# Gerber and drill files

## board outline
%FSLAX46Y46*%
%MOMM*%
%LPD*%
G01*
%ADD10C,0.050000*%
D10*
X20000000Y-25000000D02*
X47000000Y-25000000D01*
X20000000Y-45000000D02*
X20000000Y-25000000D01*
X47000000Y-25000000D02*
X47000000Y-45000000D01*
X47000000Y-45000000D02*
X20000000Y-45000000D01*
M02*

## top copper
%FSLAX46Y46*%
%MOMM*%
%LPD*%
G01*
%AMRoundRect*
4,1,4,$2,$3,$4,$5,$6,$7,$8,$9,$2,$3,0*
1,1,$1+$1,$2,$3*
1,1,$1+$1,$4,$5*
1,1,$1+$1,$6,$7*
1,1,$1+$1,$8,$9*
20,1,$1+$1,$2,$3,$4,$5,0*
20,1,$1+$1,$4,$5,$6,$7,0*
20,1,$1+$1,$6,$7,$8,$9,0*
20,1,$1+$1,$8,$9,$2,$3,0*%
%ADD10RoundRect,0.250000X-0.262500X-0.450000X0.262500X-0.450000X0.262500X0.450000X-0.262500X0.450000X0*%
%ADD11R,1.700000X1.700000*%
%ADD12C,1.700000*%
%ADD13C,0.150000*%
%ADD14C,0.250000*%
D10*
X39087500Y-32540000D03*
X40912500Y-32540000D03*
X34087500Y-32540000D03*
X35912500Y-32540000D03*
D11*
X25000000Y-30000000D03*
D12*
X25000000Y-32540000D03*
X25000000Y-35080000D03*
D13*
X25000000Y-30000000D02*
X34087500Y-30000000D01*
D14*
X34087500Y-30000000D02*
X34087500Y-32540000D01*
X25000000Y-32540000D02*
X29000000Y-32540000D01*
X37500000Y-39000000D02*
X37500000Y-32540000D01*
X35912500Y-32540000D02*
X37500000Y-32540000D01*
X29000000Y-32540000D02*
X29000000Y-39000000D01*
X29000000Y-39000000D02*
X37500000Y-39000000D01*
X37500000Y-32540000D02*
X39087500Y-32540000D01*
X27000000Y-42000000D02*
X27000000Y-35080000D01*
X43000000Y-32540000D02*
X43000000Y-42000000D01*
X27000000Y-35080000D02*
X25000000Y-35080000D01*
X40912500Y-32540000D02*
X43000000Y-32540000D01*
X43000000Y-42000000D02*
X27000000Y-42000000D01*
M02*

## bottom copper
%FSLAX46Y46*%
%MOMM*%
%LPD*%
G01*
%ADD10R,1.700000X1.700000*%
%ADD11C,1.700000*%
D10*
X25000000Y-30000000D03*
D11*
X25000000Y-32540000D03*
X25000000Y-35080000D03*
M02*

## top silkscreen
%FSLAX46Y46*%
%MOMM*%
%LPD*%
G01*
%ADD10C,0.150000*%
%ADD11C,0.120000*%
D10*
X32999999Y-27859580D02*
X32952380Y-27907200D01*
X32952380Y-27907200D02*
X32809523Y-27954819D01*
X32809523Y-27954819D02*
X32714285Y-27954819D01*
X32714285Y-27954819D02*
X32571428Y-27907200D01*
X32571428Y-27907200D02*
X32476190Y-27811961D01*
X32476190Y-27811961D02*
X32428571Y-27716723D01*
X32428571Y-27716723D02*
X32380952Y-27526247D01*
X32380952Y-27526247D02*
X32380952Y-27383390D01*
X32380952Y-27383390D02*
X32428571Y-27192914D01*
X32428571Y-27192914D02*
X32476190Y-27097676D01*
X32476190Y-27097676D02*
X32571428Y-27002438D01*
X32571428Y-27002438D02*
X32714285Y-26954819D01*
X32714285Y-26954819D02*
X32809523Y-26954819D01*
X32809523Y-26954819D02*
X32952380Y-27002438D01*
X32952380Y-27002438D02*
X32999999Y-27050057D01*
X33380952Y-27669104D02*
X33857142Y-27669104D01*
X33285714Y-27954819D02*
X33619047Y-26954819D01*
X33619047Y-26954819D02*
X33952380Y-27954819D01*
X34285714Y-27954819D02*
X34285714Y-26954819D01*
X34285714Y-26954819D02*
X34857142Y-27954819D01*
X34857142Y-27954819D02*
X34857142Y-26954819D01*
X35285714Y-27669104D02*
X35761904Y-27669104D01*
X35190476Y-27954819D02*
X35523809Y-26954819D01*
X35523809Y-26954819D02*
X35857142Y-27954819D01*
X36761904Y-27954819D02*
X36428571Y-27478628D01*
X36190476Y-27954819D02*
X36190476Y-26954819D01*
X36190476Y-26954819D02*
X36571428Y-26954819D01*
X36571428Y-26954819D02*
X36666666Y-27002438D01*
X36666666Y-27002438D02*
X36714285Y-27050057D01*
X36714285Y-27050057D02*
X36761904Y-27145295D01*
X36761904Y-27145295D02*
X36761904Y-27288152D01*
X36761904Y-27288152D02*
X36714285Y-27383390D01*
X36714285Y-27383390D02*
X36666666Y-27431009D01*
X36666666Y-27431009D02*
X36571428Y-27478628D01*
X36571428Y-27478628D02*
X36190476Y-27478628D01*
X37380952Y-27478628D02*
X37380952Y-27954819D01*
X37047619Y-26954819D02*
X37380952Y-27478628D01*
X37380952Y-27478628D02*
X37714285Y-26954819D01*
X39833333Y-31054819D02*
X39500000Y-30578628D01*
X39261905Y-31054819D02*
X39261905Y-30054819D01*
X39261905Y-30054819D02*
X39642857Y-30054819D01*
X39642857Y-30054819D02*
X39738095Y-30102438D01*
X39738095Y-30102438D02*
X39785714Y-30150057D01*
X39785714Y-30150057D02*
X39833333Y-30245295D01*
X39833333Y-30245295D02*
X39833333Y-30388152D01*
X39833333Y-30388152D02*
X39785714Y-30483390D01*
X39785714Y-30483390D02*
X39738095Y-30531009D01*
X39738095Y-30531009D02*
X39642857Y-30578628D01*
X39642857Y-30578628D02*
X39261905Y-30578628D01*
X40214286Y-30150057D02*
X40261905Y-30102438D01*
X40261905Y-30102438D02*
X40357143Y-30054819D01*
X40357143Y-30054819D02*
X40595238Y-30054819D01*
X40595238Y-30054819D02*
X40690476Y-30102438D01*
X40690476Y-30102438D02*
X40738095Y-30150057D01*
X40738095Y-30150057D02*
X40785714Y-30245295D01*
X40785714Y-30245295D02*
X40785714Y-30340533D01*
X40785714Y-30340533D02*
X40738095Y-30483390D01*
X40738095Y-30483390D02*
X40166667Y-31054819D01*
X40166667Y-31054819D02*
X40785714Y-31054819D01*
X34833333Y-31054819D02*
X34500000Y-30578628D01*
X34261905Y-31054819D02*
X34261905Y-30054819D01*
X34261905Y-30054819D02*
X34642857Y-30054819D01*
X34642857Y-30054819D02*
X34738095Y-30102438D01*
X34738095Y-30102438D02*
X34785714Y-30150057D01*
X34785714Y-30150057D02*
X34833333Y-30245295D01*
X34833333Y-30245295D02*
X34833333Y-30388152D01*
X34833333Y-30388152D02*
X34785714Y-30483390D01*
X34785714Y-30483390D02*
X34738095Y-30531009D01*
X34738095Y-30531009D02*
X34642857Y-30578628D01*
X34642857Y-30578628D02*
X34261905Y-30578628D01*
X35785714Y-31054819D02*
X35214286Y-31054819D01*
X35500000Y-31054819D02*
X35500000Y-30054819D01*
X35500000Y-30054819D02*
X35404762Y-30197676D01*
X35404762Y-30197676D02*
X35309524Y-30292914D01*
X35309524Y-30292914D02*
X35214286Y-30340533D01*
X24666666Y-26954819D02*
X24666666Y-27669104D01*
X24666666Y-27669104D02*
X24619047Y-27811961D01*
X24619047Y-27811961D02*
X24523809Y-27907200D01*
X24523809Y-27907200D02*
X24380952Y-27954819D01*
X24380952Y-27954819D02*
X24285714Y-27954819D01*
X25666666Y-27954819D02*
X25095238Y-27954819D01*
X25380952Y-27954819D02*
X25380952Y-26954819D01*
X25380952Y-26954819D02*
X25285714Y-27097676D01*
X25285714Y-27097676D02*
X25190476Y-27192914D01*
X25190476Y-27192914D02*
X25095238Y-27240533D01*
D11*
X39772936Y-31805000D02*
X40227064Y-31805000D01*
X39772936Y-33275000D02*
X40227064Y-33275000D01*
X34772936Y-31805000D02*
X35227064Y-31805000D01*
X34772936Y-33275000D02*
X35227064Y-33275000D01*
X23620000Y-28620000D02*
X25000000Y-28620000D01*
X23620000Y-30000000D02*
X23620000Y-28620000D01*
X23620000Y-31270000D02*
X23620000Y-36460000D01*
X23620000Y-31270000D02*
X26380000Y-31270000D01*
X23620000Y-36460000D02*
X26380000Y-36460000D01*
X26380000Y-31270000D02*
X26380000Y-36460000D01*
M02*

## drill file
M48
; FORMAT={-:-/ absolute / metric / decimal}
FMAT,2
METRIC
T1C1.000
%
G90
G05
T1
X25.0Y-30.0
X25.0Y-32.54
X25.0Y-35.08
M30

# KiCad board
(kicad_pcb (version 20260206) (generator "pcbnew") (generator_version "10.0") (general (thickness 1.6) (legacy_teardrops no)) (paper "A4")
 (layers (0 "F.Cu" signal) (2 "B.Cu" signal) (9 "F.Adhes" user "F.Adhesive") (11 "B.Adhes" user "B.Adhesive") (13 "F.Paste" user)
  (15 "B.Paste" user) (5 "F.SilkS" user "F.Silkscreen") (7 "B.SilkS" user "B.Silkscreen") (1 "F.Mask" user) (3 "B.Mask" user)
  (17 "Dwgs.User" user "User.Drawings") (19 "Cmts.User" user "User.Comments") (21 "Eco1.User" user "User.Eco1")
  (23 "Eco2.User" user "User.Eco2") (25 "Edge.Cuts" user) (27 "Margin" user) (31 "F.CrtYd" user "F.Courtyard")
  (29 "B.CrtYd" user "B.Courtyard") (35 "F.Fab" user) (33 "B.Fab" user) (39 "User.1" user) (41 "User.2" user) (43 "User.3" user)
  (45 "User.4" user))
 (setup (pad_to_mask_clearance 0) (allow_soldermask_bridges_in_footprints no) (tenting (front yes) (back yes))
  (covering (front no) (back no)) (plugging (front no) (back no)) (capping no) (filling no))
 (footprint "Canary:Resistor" (layer "F.Cu") (at 40 32.54)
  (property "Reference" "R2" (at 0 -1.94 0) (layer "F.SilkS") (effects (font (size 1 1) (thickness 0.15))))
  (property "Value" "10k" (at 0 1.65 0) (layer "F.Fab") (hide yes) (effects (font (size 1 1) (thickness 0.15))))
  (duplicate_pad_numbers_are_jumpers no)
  (fp_line (start -0.227064 -0.735) (end 0.227064 -0.735) (stroke (width 0.12) (type solid)) (layer "F.SilkS"))
  (fp_line (start -0.227064 0.735) (end 0.227064 0.735) (stroke (width 0.12) (type solid)) (layer "F.SilkS"))
  (pad "1" smd roundrect (at -0.9125 0) (size 1.025 1.4) (layers "F.Cu" "F.Mask" "F.Paste") (roundrect_rratio 0.243902) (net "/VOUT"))
  (pad "2" smd roundrect (at 0.9125 0) (size 1.025 1.4) (layers "F.Cu" "F.Mask" "F.Paste") (roundrect_rratio 0.243902) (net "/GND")))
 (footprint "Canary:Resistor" (layer "F.Cu") (at 35 32.54)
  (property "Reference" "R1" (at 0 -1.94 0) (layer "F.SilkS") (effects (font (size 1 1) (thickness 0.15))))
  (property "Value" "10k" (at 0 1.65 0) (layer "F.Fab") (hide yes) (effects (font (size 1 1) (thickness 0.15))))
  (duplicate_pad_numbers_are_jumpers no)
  (fp_line (start -0.227064 -0.735) (end 0.227064 -0.735) (stroke (width 0.12) (type solid)) (layer "F.SilkS"))
  (fp_line (start -0.227064 0.735) (end 0.227064 0.735) (stroke (width 0.12) (type solid)) (layer "F.SilkS"))
  (pad "1" smd roundrect (at -0.9125 0) (size 1.025 1.4) (layers "F.Cu" "F.Mask" "F.Paste") (roundrect_rratio 0.243902) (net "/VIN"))
  (pad "2" smd roundrect (at 0.9125 0) (size 1.025 1.4) (layers "F.Cu" "F.Mask" "F.Paste") (roundrect_rratio 0.243902) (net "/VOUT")))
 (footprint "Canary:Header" (layer "F.Cu") (at 25 30)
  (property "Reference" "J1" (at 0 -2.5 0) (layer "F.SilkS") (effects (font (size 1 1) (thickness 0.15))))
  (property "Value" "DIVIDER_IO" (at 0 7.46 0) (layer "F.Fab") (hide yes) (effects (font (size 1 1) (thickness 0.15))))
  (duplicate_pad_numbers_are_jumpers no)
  (fp_line (start -1.38 -1.38) (end 0 -1.38) (stroke (width 0.12) (type solid)) (layer "F.SilkS"))
  (fp_line (start -1.38 0) (end -1.38 -1.38) (stroke (width 0.12) (type solid)) (layer "F.SilkS"))
  (fp_line (start -1.38 1.27) (end -1.38 6.46) (stroke (width 0.12) (type solid)) (layer "F.SilkS"))
  (fp_line (start -1.38 1.27) (end 1.38 1.27) (stroke (width 0.12) (type solid)) (layer "F.SilkS"))
  (fp_line (start -1.38 6.46) (end 1.38 6.46) (stroke (width 0.12) (type solid)) (layer "F.SilkS"))
  (fp_line (start 1.38 1.27) (end 1.38 6.46) (stroke (width 0.12) (type solid)) (layer "F.SilkS"))
  (pad "1" thru_hole rect (at 0 0) (size 1.7 1.7) (drill 1) (layers "*.Cu" "*.Mask") (remove_unused_layers no) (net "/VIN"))
  (pad "2" thru_hole circle (at 0 2.54) (size 1.7 1.7) (drill 1) (layers "*.Cu" "*.Mask") (remove_unused_layers no) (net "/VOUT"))
  (pad "3" thru_hole circle (at 0 5.08) (size 1.7 1.7) (drill 1) (layers "*.Cu" "*.Mask") (remove_unused_layers no) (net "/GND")))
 (gr_line (start 20 25) (end 47 25) (stroke (width 0.05) (type default)) (layer "Edge.Cuts"))
 (gr_line (start 20 45) (end 20 25) (stroke (width 0.05) (type default)) (layer "Edge.Cuts"))
 (gr_line (start 47 25) (end 47 45) (stroke (width 0.05) (type default)) (layer "Edge.Cuts"))
 (gr_line (start 47 45) (end 20 45) (stroke (width 0.05) (type default)) (layer "Edge.Cuts"))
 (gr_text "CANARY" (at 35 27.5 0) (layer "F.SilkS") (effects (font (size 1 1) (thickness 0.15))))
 (segment (start 25 30) (end 34.0875 30) (width 0.15) (layer "F.Cu") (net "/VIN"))
 (segment (start 34.0875 30) (end 34.0875 32.54) (width 0.25) (layer "F.Cu") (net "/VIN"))
 (segment (start 25 32.54) (end 29 32.54) (width 0.25) (layer "F.Cu") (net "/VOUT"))
 (segment (start 37.5 39) (end 37.5 32.54) (width 0.25) (layer "F.Cu") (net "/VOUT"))
 (segment (start 35.9125 32.54) (end 37.5 32.54) (width 0.25) (layer "F.Cu") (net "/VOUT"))
 (segment (start 29 32.54) (end 29 39) (width 0.25) (layer "F.Cu") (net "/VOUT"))
 (segment (start 29 39) (end 37.5 39) (width 0.25) (layer "F.Cu") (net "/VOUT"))
 (segment (start 37.5 32.54) (end 39.0875 32.54) (width 0.25) (layer "F.Cu") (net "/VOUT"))
 (segment (start 27 42) (end 27 35.08) (width 0.25) (layer "F.Cu") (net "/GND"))
 (segment (start 43 32.54) (end 43 42) (width 0.25) (layer "F.Cu") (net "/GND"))
 (segment (start 27 35.08) (end 25 35.08) (width 0.25) (layer "F.Cu") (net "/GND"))
 (segment (start 40.9125 32.54) (end 43 32.54) (width 0.25) (layer "F.Cu") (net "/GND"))
 (segment (start 43 42) (end 27 42) (width 0.25) (layer "F.Cu") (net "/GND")))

